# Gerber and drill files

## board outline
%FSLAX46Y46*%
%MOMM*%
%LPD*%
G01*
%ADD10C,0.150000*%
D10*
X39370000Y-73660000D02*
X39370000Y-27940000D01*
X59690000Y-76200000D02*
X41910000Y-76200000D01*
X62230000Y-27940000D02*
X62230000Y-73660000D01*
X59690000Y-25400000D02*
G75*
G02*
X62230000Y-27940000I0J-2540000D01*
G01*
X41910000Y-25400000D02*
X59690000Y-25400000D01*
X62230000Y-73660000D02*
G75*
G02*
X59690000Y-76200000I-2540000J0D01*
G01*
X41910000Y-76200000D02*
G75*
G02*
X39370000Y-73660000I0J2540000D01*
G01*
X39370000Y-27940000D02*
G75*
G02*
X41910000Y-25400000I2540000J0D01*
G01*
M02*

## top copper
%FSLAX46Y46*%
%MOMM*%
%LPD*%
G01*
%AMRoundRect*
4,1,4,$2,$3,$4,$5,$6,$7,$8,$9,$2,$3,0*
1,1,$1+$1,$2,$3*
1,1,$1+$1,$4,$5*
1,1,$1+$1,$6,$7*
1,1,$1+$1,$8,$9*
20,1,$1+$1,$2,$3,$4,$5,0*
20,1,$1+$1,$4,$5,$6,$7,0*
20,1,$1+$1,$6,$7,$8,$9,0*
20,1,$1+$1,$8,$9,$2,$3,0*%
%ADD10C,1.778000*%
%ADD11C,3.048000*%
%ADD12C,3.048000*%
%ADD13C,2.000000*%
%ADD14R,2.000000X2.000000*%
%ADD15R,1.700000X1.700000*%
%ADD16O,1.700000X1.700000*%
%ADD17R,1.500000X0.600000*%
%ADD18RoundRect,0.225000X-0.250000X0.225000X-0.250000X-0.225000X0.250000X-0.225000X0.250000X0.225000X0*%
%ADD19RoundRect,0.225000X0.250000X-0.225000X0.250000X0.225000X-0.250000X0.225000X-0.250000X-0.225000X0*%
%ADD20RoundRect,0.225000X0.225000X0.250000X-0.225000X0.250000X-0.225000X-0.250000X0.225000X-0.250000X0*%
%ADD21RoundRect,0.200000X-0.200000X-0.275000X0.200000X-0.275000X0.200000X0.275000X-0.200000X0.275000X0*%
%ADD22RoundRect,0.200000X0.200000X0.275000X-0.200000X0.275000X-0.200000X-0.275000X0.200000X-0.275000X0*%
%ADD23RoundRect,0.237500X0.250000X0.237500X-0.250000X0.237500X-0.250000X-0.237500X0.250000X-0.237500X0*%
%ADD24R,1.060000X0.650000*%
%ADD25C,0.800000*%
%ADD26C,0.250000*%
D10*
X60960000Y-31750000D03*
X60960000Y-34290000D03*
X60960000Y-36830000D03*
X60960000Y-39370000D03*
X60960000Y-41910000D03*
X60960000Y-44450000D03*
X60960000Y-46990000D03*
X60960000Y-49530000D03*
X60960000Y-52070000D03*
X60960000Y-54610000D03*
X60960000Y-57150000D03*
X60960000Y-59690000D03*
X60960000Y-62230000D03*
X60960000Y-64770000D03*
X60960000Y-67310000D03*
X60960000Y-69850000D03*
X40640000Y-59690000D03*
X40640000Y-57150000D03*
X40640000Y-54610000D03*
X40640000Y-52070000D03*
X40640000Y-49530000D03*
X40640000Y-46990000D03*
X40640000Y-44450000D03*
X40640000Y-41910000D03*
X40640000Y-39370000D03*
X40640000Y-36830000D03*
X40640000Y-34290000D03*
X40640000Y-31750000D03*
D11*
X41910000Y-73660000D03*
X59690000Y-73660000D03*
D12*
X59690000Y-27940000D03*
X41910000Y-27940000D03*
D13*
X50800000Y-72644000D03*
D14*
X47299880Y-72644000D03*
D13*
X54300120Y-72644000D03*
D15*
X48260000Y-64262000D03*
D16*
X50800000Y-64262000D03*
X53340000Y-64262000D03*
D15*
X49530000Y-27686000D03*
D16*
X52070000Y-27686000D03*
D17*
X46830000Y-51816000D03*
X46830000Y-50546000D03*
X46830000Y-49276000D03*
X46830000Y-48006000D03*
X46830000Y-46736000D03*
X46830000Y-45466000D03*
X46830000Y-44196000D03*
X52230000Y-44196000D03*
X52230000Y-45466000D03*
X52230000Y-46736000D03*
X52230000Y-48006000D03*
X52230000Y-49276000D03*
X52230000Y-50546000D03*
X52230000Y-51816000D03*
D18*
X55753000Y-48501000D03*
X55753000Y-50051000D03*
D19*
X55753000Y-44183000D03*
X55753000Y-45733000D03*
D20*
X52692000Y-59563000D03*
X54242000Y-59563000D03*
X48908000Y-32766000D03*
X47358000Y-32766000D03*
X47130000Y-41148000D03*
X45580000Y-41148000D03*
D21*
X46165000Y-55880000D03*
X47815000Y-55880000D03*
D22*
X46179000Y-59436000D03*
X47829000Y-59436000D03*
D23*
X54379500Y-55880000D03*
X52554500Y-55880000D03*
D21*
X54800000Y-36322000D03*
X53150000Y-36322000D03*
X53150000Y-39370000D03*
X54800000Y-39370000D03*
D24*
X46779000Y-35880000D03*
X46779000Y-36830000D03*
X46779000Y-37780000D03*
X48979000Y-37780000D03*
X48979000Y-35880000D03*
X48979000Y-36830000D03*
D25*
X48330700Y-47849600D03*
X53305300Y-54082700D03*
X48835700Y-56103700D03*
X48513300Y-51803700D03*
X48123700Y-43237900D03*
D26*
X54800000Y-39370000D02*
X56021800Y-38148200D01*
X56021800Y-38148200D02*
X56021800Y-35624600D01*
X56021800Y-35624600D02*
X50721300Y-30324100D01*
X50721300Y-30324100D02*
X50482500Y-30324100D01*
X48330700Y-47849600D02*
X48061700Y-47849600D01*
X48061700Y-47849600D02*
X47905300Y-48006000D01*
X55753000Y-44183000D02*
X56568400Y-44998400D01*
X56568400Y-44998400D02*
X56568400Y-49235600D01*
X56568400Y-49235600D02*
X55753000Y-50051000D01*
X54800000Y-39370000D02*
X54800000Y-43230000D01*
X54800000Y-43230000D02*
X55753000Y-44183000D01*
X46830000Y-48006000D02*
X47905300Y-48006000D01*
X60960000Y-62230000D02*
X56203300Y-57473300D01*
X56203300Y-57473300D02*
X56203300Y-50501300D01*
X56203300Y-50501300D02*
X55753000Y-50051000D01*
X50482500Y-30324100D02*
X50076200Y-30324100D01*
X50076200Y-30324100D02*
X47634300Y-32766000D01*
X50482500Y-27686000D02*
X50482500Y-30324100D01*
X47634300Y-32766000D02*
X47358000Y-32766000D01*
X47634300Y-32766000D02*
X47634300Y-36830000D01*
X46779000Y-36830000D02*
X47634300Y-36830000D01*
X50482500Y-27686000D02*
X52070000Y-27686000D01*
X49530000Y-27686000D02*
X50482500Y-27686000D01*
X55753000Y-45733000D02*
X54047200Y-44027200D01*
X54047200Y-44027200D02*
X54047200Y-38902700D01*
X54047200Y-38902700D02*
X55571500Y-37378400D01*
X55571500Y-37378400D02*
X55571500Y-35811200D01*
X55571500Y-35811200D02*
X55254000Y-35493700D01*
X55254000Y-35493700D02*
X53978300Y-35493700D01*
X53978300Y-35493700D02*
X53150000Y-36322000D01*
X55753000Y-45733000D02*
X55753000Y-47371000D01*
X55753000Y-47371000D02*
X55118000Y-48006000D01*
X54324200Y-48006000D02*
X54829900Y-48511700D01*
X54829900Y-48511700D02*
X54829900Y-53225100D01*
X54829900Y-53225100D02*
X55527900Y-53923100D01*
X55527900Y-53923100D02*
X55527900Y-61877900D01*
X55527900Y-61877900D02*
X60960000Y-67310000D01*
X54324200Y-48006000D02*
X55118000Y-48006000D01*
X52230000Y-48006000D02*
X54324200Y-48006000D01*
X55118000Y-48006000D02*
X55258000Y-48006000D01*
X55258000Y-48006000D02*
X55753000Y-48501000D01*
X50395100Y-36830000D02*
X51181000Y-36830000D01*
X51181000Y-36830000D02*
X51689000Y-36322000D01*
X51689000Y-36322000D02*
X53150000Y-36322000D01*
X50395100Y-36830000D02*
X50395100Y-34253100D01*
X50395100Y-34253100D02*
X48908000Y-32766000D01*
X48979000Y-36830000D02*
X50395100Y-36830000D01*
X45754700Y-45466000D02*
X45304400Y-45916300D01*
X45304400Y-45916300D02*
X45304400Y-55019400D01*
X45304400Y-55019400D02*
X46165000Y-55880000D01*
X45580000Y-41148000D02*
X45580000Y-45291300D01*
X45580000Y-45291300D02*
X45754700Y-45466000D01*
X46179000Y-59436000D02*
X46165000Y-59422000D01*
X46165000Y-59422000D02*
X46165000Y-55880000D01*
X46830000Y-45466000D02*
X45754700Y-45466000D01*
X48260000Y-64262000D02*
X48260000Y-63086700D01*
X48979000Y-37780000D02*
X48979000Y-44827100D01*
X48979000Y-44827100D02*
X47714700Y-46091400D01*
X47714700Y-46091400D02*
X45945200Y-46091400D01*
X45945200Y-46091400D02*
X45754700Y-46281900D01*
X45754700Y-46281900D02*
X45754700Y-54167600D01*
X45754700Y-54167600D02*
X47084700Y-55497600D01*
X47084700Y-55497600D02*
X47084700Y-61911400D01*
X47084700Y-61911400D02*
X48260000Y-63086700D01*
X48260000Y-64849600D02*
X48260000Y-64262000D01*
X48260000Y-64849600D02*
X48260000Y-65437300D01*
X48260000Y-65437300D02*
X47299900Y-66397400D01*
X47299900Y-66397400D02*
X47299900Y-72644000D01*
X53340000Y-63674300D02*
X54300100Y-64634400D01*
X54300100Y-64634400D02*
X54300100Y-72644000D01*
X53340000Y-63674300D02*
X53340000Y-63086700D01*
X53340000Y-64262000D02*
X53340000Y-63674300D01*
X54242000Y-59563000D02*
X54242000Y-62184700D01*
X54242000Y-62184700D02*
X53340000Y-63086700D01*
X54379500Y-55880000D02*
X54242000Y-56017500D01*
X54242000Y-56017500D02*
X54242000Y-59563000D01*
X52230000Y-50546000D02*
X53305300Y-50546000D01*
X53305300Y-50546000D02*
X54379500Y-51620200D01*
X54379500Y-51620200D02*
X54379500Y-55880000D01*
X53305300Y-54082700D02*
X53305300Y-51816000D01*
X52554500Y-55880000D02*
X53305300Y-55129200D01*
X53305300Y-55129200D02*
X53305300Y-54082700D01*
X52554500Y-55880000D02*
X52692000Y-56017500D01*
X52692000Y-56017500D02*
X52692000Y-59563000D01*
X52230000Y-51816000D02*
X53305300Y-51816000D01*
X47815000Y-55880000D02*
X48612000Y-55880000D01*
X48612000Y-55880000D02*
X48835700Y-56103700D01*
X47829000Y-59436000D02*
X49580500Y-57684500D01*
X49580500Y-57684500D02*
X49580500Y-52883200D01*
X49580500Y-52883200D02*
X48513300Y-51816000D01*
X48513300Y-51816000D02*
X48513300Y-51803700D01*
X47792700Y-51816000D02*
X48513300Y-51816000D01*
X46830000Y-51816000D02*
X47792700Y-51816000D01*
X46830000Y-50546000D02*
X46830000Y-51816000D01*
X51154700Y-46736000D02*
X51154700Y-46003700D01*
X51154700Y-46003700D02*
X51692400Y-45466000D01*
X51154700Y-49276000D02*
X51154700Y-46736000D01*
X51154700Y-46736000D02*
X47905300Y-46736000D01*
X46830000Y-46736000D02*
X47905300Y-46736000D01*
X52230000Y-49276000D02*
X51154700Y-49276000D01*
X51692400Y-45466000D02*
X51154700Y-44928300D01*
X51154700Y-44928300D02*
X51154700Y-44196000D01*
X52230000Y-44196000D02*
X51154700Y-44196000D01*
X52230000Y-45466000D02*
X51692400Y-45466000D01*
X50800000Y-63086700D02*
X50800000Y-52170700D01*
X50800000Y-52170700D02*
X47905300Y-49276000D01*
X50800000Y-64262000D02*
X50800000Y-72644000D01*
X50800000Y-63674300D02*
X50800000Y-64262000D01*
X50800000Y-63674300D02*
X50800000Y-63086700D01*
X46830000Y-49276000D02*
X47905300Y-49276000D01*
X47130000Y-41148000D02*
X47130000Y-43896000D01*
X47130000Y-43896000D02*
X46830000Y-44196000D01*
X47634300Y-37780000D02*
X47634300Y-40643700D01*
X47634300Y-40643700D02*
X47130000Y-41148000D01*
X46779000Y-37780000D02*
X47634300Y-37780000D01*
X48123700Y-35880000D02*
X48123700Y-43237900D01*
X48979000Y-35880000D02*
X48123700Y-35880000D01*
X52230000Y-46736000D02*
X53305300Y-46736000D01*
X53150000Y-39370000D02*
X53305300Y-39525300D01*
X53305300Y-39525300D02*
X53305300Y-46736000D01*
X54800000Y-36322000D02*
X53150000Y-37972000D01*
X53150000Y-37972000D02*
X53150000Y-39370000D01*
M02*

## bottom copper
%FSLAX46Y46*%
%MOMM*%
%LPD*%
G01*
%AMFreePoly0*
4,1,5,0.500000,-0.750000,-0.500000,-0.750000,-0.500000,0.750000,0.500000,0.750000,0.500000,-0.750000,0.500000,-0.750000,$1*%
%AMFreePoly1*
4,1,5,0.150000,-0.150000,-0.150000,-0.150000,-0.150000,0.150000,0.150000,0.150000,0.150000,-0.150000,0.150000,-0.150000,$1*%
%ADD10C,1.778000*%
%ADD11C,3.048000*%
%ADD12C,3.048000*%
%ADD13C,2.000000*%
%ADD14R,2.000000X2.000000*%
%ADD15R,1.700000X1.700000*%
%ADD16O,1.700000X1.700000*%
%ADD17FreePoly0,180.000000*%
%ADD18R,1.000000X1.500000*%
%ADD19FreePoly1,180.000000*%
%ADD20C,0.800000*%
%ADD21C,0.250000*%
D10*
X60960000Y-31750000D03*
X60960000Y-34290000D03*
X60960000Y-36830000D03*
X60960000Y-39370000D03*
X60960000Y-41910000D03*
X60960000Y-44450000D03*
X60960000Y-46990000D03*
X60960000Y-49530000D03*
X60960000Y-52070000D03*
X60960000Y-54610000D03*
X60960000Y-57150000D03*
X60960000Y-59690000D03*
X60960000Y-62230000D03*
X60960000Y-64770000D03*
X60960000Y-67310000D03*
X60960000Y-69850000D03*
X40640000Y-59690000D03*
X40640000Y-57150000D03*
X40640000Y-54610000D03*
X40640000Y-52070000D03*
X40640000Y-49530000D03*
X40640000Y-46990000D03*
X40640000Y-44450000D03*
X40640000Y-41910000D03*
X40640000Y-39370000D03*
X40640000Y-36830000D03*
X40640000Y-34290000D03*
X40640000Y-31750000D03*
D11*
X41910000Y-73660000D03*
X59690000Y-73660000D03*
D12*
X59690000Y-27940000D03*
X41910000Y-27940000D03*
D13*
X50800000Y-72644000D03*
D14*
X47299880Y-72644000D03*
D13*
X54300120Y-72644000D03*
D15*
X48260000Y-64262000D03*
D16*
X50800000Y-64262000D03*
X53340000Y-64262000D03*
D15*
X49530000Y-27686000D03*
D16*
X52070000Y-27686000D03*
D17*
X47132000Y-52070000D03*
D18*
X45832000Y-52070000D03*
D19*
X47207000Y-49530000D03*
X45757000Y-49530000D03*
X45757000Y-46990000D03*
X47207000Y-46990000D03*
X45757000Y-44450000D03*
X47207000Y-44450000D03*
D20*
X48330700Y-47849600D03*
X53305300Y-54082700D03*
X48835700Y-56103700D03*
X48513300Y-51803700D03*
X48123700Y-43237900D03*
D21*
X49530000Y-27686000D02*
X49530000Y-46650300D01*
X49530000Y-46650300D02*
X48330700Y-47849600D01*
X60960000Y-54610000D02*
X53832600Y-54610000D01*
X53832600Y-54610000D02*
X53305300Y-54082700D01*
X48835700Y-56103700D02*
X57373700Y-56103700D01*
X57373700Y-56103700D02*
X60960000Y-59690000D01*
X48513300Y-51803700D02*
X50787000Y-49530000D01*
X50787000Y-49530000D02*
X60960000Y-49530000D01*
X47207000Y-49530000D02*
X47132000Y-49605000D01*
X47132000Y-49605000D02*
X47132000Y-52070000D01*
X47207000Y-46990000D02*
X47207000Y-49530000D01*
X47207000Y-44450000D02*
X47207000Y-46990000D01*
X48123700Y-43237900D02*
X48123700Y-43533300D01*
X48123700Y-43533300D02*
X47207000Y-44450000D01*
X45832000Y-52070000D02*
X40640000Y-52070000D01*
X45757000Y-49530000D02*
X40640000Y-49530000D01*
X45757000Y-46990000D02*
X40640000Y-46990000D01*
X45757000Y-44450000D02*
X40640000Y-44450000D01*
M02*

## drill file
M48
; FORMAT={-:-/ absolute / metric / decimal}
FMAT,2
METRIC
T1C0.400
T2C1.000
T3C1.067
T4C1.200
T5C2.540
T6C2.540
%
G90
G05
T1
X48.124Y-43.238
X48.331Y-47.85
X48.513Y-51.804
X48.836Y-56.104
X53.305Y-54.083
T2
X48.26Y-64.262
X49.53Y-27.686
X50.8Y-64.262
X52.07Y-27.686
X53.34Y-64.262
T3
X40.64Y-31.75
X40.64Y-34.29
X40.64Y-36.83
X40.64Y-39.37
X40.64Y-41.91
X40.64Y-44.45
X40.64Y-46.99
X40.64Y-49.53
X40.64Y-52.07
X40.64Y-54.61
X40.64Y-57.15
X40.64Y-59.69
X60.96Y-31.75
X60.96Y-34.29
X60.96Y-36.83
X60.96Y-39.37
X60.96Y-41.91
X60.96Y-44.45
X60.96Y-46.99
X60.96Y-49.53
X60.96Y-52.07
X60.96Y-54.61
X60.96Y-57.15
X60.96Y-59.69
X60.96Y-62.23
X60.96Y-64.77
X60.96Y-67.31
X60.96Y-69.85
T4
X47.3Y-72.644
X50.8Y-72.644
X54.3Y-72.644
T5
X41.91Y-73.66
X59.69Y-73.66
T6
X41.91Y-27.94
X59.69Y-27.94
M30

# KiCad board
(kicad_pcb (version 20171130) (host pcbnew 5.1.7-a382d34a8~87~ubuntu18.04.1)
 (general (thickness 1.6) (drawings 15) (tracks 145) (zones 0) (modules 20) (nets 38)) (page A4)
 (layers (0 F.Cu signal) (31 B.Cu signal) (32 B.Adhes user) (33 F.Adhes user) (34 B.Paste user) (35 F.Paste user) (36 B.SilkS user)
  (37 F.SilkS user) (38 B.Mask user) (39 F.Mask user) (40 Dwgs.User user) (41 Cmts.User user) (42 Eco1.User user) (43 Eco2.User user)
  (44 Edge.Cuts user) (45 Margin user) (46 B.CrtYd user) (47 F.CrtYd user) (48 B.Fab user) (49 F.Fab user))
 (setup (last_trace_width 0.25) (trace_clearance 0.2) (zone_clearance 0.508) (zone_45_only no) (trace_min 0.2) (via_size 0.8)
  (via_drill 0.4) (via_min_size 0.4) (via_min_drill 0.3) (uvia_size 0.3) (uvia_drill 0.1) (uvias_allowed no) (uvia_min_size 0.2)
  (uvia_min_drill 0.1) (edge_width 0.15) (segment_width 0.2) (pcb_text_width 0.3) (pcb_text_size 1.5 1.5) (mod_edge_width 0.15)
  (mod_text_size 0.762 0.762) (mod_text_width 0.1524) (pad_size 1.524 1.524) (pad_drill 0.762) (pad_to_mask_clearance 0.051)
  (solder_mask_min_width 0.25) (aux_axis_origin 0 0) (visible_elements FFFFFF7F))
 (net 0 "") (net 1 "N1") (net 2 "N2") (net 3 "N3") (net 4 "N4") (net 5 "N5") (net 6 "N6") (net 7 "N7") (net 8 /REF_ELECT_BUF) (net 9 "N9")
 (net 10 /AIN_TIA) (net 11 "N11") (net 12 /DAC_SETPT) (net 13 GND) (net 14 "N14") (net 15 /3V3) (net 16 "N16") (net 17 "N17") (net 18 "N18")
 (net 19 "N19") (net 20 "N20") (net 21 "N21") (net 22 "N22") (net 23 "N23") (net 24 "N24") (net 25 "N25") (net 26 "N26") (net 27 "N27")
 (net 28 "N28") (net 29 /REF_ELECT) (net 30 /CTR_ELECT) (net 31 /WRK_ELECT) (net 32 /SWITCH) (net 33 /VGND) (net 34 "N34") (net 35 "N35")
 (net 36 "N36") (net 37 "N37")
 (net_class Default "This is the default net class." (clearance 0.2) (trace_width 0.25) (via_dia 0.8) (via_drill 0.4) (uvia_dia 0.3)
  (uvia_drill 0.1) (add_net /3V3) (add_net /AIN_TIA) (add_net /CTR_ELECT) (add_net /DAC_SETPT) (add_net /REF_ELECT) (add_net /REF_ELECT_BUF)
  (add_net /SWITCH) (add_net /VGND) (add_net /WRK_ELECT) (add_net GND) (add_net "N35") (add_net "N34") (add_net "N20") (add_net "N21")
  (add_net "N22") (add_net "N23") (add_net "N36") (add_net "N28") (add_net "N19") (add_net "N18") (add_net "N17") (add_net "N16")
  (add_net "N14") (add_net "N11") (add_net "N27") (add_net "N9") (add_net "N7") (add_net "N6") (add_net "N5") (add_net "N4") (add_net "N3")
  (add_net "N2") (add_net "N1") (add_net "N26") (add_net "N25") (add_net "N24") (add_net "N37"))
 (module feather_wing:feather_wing (layer F.Cu) (at 50.8 50.8)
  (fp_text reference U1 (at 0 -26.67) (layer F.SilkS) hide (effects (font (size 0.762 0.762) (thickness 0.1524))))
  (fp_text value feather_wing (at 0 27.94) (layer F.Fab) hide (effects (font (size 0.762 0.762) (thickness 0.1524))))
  (pad 28 thru_hole circle (at 10.16 -19.05) (size 1.778 1.778) (drill 1.0668) (layers *.Cu *.Mask) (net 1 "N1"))
  (pad 27 thru_hole circle (at 10.16 -16.51) (size 1.778 1.778) (drill 1.0668) (layers *.Cu *.Mask) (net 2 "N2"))
  (pad 26 thru_hole circle (at 10.16 -13.97) (size 1.778 1.778) (drill 1.0668) (layers *.Cu *.Mask) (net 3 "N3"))
  (pad 25 thru_hole circle (at 10.16 -11.43) (size 1.778 1.778) (drill 1.0668) (layers *.Cu *.Mask) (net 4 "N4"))
  (pad 24 thru_hole circle (at 10.16 -8.89) (size 1.778 1.778) (drill 1.0668) (layers *.Cu *.Mask) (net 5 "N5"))
  (pad 23 thru_hole circle (at 10.16 -6.35) (size 1.778 1.778) (drill 1.0668) (layers *.Cu *.Mask) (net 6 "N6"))
  (pad 22 thru_hole circle (at 10.16 -3.81) (size 1.778 1.778) (drill 1.0668) (layers *.Cu *.Mask) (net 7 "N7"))
  (pad 21 thru_hole circle (at 10.16 -1.27) (size 1.778 1.778) (drill 1.0668) (layers *.Cu *.Mask) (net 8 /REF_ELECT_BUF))
  (pad 20 thru_hole circle (at 10.16 1.27) (size 1.778 1.778) (drill 1.0668) (layers *.Cu *.Mask) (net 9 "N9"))
  (pad 19 thru_hole circle (at 10.16 3.81) (size 1.778 1.778) (drill 1.0668) (layers *.Cu *.Mask) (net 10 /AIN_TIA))
  (pad 18 thru_hole circle (at 10.16 6.35) (size 1.778 1.778) (drill 1.0668) (layers *.Cu *.Mask) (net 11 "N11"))
  (pad 17 thru_hole circle (at 10.16 8.89) (size 1.778 1.778) (drill 1.0668) (layers *.Cu *.Mask) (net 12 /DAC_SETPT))
  (pad 16 thru_hole circle (at 10.16 11.43) (size 1.778 1.778) (drill 1.0668) (layers *.Cu *.Mask) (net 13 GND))
  (pad 15 thru_hole circle (at 10.16 13.97) (size 1.778 1.778) (drill 1.0668) (layers *.Cu *.Mask) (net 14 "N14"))
  (pad 14 thru_hole circle (at 10.16 16.51) (size 1.778 1.778) (drill 1.0668) (layers *.Cu *.Mask) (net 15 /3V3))
  (pad 13 thru_hole circle (at 10.16 19.05) (size 1.778 1.778) (drill 1.0668) (layers *.Cu *.Mask) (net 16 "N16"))
  (pad 12 thru_hole circle (at -10.16 8.89) (size 1.778 1.778) (drill 1.0668) (layers *.Cu *.Mask) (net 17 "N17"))
  (pad 11 thru_hole circle (at -10.16 6.35) (size 1.778 1.778) (drill 1.0668) (layers *.Cu *.Mask) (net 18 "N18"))
  (pad 10 thru_hole circle (at -10.16 3.81) (size 1.778 1.778) (drill 1.0668) (layers *.Cu *.Mask) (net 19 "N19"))
  (pad 9 thru_hole circle (at -10.16 1.27) (size 1.778 1.778) (drill 1.0668) (layers *.Cu *.Mask) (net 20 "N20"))
  (pad 8 thru_hole circle (at -10.16 -1.27) (size 1.778 1.778) (drill 1.0668) (layers *.Cu *.Mask) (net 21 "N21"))
  (pad 7 thru_hole circle (at -10.16 -3.81) (size 1.778 1.778) (drill 1.0668) (layers *.Cu *.Mask) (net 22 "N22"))
  (pad 6 thru_hole circle (at -10.16 -6.35) (size 1.778 1.778) (drill 1.0668) (layers *.Cu *.Mask) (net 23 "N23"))
  (pad 5 thru_hole circle (at -10.16 -8.89) (size 1.778 1.778) (drill 1.0668) (layers *.Cu *.Mask) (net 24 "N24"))
  (pad 4 thru_hole circle (at -10.16 -11.43) (size 1.778 1.778) (drill 1.0668) (layers *.Cu *.Mask) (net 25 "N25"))
  (pad 3 thru_hole circle (at -10.16 -13.97) (size 1.778 1.778) (drill 1.0668) (layers *.Cu *.Mask) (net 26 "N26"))
  (pad 2 thru_hole circle (at -10.16 -16.51) (size 1.778 1.778) (drill 1.0668) (layers *.Cu *.Mask) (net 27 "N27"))
  (pad 1 thru_hole circle (at -10.16 -19.05) (size 1.778 1.778) (drill 1.0668) (layers *.Cu *.Mask) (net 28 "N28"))
  (pad "" thru_hole circle (at -8.89 22.86) (size 3.048 3.048) (drill 2.54) (layers *.Cu *.Mask))
  (pad "" thru_hole circle (at 8.89 22.86) (size 3.048 3.048) (drill 2.54) (layers *.Cu *.Mask))
  (pad "" np_thru_hole circle (at 8.89 -22.86) (size 3.048 3.048) (drill 2.54) (layers *.Cu *.Mask))
  (pad "" np_thru_hole circle (at -8.89 -22.86) (size 3.048 3.048) (drill 2.54) (layers *.Cu *.Mask)))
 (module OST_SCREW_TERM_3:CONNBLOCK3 (layer F.Cu) (at 50.8 72.644)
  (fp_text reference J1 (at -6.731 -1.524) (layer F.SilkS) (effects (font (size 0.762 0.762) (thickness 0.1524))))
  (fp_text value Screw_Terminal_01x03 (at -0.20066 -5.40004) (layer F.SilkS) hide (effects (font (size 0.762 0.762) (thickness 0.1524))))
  (pad 2 thru_hole circle (at 0 0) (size 2 2) (drill 1.2) (layers *.Cu *.Mask) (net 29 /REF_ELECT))
  (pad 1 thru_hole rect (at -3.50012 0) (size 2 2) (drill 1.2) (layers *.Cu *.Mask) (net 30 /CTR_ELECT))
  (pad 3 thru_hole circle (at 3.50012 0) (size 2 2) (drill 1.2) (layers *.Cu *.Mask) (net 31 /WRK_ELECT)))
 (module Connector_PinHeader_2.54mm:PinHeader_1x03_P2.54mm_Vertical (layer F.Cu) (at 48.26 64.262 90)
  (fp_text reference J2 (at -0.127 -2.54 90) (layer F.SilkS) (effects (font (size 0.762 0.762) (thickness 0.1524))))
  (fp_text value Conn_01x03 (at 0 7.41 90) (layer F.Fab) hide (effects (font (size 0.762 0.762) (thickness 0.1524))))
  (pad 1 thru_hole rect (at 0 0 90) (size 1.7 1.7) (drill 1) (layers *.Cu *.Mask) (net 30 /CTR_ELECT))
  (pad 2 thru_hole oval (at 0 2.54 90) (size 1.7 1.7) (drill 1) (layers *.Cu *.Mask) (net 29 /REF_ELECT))
  (pad 3 thru_hole oval (at 0 5.08 90) (size 1.7 1.7) (drill 1) (layers *.Cu *.Mask) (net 31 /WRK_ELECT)))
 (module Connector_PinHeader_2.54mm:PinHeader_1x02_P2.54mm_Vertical (layer F.Cu) (at 49.53 27.686 90)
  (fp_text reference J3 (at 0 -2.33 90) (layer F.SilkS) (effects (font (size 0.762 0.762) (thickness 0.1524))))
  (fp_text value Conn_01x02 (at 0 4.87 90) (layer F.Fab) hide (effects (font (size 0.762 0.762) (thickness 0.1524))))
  (pad 1 thru_hole rect (at 0 0 90) (size 1.7 1.7) (drill 1) (layers *.Cu *.Mask) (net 13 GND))
  (pad 2 thru_hole oval (at 0 2.54 90) (size 1.7 1.7) (drill 1) (layers *.Cu *.Mask) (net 13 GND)))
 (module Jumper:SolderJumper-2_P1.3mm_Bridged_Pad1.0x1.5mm (layer B.Cu) (at 46.482 52.07 180)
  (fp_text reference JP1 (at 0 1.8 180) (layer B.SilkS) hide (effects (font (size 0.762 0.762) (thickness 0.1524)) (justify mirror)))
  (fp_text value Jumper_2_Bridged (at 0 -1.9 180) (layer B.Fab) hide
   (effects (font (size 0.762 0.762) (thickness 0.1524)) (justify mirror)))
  (pad 1 smd custom (at -0.65 0 180) (size 1 1.5) (layers B.Cu B.Mask) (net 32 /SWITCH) (options (clearance outline) (anchor rect))
   (primitives))
  (pad 2 smd rect (at 0.65 0 180) (size 1 1.5) (layers B.Cu B.Mask) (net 20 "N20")))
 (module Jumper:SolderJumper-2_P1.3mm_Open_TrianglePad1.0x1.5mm (layer B.Cu) (at 46.482 49.53 180)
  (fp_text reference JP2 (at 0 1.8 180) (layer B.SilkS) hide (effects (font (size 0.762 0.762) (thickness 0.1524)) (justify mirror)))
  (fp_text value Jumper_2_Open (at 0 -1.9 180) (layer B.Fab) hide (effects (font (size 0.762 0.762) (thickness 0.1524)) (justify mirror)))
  (pad 1 smd custom (at -0.725 0 180) (size 0.3 0.3) (layers B.Cu B.Mask) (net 32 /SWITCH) (zone_connect 0)
   (options (clearance outline) (anchor rect)) (primitives))
  (pad 2 smd custom (at 0.725 0 180) (size 0.3 0.3) (layers B.Cu B.Mask) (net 21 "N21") (zone_connect 0)
   (options (clearance outline) (anchor rect)) (primitives)))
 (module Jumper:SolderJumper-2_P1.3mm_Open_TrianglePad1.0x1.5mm (layer B.Cu) (at 46.482 46.99 180)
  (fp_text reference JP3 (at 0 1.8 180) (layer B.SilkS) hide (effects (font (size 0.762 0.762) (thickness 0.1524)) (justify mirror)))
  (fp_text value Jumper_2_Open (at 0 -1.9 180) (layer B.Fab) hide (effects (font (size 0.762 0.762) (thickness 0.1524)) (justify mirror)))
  (pad 2 smd custom (at 0.725 0 180) (size 0.3 0.3) (layers B.Cu B.Mask) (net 22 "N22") (zone_connect 0)
   (options (clearance outline) (anchor rect)) (primitives))
  (pad 1 smd custom (at -0.725 0 180) (size 0.3 0.3) (layers B.Cu B.Mask) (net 32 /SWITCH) (zone_connect 0)
   (options (clearance outline) (anchor rect)) (primitives)))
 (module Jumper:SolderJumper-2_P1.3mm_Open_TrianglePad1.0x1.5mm (layer B.Cu) (at 46.482 44.45 180)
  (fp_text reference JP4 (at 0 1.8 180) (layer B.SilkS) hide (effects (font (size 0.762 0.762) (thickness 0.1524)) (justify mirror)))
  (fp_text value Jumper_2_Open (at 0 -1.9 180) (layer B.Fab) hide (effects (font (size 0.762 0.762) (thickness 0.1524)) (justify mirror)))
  (pad 2 smd custom (at 0.725 0 180) (size 0.3 0.3) (layers B.Cu B.Mask) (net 23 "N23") (zone_connect 0)
   (options (clearance outline) (anchor rect)) (primitives))
  (pad 1 smd custom (at -0.725 0 180) (size 0.3 0.3) (layers B.Cu B.Mask) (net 32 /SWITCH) (zone_connect 0)
   (options (clearance outline) (anchor rect)) (primitives)))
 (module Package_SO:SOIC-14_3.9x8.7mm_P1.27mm (layer F.Cu) (at 49.53 48.006 180)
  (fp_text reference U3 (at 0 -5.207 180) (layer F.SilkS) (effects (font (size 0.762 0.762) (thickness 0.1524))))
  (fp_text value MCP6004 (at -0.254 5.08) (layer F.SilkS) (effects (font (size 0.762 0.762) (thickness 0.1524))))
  (pad 14 smd rect (at 2.7 -3.81 180) (size 1.5 0.6) (layers F.Cu F.Paste F.Mask) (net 8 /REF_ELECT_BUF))
  (pad 13 smd rect (at 2.7 -2.54 180) (size 1.5 0.6) (layers F.Cu F.Paste F.Mask) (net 8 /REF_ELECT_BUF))
  (pad 12 smd rect (at 2.7 -1.27 180) (size 1.5 0.6) (layers F.Cu F.Paste F.Mask) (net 29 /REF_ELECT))
  (pad 11 smd rect (at 2.7 0 180) (size 1.5 0.6) (layers F.Cu F.Paste F.Mask) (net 13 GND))
  (pad 10 smd rect (at 2.7 1.27 180) (size 1.5 0.6) (layers F.Cu F.Paste F.Mask) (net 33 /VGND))
  (pad 9 smd rect (at 2.7 2.54 180) (size 1.5 0.6) (layers F.Cu F.Paste F.Mask) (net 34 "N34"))
  (pad 8 smd rect (at 2.7 3.81 180) (size 1.5 0.6) (layers F.Cu F.Paste F.Mask) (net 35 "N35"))
  (pad 7 smd rect (at -2.7 3.81 180) (size 1.5 0.6) (layers F.Cu F.Paste F.Mask) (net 33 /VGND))
  (pad 6 smd rect (at -2.7 2.54 180) (size 1.5 0.6) (layers F.Cu F.Paste F.Mask) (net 33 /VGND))
  (pad 5 smd rect (at -2.7 1.27 180) (size 1.5 0.6) (layers F.Cu F.Paste F.Mask) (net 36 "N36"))
  (pad 4 smd rect (at -2.7 0 180) (size 1.5 0.6) (layers F.Cu F.Paste F.Mask) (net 15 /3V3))
  (pad 3 smd rect (at -2.7 -1.27 180) (size 1.5 0.6) (layers F.Cu F.Paste F.Mask) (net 33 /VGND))
  (pad 2 smd rect (at -2.7 -2.54 180) (size 1.5 0.6) (layers F.Cu F.Paste F.Mask) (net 31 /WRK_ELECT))
  (pad 1 smd rect (at -2.7 -3.81 180) (size 1.5 0.6) (layers F.Cu F.Paste F.Mask) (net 10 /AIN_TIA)))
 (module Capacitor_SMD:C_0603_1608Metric (layer F.Cu) (at 55.753 49.276 270)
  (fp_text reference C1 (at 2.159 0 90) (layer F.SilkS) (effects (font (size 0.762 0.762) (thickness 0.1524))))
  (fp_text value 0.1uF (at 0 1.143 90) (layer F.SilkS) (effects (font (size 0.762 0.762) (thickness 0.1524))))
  (pad 1 smd roundrect (at -0.775 0 270) (size 0.9 0.95) (layers F.Cu F.Paste F.Mask) (roundrect_rratio 0.25) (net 15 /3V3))
  (pad 2 smd roundrect (at 0.775 0 270) (size 0.9 0.95) (layers F.Cu F.Paste F.Mask) (roundrect_rratio 0.25) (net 13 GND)))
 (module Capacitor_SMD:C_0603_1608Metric (layer F.Cu) (at 55.753 44.958 90)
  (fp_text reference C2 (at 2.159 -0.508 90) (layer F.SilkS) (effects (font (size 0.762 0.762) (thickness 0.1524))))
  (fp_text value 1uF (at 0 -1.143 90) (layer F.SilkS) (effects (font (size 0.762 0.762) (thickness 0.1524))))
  (pad 2 smd roundrect (at 0.775 0 90) (size 0.9 0.95) (layers F.Cu F.Paste F.Mask) (roundrect_rratio 0.25) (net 13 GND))
  (pad 1 smd roundrect (at -0.775 0 90) (size 0.9 0.95) (layers F.Cu F.Paste F.Mask) (roundrect_rratio 0.25) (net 15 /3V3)))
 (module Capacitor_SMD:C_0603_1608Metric (layer F.Cu) (at 53.467 59.563 180)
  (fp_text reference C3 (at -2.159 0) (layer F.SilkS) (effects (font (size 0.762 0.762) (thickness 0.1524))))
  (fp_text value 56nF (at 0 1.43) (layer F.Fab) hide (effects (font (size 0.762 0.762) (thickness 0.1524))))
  (pad 2 smd roundrect (at 0.775 0 180) (size 0.9 0.95) (layers F.Cu F.Paste F.Mask) (roundrect_rratio 0.25) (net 10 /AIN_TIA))
  (pad 1 smd roundrect (at -0.775 0 180) (size 0.9 0.95) (layers F.Cu F.Paste F.Mask) (roundrect_rratio 0.25) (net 31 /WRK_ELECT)))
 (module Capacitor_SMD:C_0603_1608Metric (layer F.Cu) (at 48.133 32.766 180)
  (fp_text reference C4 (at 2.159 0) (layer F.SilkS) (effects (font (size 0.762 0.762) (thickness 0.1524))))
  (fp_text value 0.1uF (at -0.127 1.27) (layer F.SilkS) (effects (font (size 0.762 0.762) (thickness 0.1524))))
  (pad 1 smd roundrect (at -0.775 0 180) (size 0.9 0.95) (layers F.Cu F.Paste F.Mask) (roundrect_rratio 0.25) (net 15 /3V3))
  (pad 2 smd roundrect (at 0.775 0 180) (size 0.9 0.95) (layers F.Cu F.Paste F.Mask) (roundrect_rratio 0.25) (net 13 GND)))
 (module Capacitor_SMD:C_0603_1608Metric (layer F.Cu) (at 46.355 41.148 180)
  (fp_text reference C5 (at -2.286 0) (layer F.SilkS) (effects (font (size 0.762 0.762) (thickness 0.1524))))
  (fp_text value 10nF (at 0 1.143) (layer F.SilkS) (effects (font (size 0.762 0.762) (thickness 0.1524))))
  (pad 1 smd roundrect (at -0.775 0 180) (size 0.9 0.95) (layers F.Cu F.Paste F.Mask) (roundrect_rratio 0.25) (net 35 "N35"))
  (pad 2 smd roundrect (at 0.775 0 180) (size 0.9 0.95) (layers F.Cu F.Paste F.Mask) (roundrect_rratio 0.25) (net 34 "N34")))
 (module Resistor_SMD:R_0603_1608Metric (layer F.Cu) (at 46.99 55.88)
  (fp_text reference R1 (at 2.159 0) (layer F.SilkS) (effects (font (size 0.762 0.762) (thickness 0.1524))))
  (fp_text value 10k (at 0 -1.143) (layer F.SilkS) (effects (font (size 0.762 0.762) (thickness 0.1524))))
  (pad 1 smd roundrect (at -0.825 0) (size 0.8 0.95) (layers F.Cu F.Paste F.Mask) (roundrect_rratio 0.25) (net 34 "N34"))
  (pad 2 smd roundrect (at 0.825 0) (size 0.8 0.95) (layers F.Cu F.Paste F.Mask) (roundrect_rratio 0.25) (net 12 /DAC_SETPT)))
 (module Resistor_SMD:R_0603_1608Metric (layer F.Cu) (at 47.004 59.436 180)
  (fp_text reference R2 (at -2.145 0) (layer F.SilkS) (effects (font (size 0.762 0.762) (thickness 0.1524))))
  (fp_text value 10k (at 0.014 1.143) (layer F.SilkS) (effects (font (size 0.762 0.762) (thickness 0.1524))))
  (pad 2 smd roundrect (at 0.825 0 180) (size 0.8 0.95) (layers F.Cu F.Paste F.Mask) (roundrect_rratio 0.25) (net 34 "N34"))
  (pad 1 smd roundrect (at -0.825 0 180) (size 0.8 0.95) (layers F.Cu F.Paste F.Mask) (roundrect_rratio 0.25) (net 8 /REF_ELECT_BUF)))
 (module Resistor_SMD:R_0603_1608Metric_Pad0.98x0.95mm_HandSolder (layer F.Cu) (at 53.467 55.88 180)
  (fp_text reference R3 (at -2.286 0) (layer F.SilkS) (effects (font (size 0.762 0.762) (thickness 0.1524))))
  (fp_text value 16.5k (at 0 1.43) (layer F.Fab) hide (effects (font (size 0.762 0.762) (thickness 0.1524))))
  (pad 1 smd roundrect (at -0.9125 0 180) (size 0.975 0.95) (layers F.Cu F.Paste F.Mask) (roundrect_rratio 0.25) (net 31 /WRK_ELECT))
  (pad 2 smd roundrect (at 0.9125 0 180) (size 0.975 0.95) (layers F.Cu F.Paste F.Mask) (roundrect_rratio 0.25) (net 10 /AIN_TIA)))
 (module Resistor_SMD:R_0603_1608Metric (layer F.Cu) (at 53.975 36.322)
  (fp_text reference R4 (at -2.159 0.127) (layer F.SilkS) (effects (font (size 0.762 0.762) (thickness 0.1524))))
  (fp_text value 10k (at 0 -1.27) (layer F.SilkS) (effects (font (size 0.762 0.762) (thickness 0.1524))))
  (pad 2 smd roundrect (at 0.825 0) (size 0.8 0.95) (layers F.Cu F.Paste F.Mask) (roundrect_rratio 0.25) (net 36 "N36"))
  (pad 1 smd roundrect (at -0.825 0) (size 0.8 0.95) (layers F.Cu F.Paste F.Mask) (roundrect_rratio 0.25) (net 15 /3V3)))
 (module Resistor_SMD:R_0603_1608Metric (layer F.Cu) (at 53.975 39.37)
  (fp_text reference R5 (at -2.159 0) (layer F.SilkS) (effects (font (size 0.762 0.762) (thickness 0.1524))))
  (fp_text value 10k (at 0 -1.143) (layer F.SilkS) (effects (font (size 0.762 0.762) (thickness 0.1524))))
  (pad 1 smd roundrect (at -0.825 0) (size 0.8 0.95) (layers F.Cu F.Paste F.Mask) (roundrect_rratio 0.25) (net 36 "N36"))
  (pad 2 smd roundrect (at 0.825 0) (size 0.8 0.95) (layers F.Cu F.Paste F.Mask) (roundrect_rratio 0.25) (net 13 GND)))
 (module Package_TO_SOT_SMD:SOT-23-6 (layer F.Cu) (at 47.879 36.83)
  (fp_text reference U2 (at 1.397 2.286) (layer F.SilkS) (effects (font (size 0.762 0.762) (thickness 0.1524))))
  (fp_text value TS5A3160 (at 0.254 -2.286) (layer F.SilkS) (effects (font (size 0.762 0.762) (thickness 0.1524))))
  (pad 1 smd rect (at -1.1 -0.95) (size 1.06 0.65) (layers F.Cu F.Paste F.Mask) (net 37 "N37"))
  (pad 2 smd rect (at -1.1 0) (size 1.06 0.65) (layers F.Cu F.Paste F.Mask) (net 13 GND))
  (pad 3 smd rect (at -1.1 0.95) (size 1.06 0.65) (layers F.Cu F.Paste F.Mask) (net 35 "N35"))
  (pad 4 smd rect (at 1.1 0.95) (size 1.06 0.65) (layers F.Cu F.Paste F.Mask) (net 30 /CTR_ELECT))
  (pad 6 smd rect (at 1.1 -0.95) (size 1.06 0.65) (layers F.Cu F.Paste F.Mask) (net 32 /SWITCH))
  (pad 5 smd rect (at 1.1 0) (size 1.06 0.65) (layers F.Cu F.Paste F.Mask) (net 15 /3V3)))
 (gr_line (start 39.37 73.66) (end 39.37 27.94) (layer Edge.Cuts) (width 0.15))
 (gr_line (start 59.69 76.2) (end 41.91 76.2) (layer Edge.Cuts) (width 0.15))
 (gr_line (start 62.23 27.94) (end 62.23 73.66) (layer Edge.Cuts) (width 0.15))
 (gr_arc (start 59.69 27.94) (end 62.23 27.94) (angle -90) (layer Edge.Cuts) (width 0.15))
 (gr_line (start 41.91 25.4) (end 59.69 25.4) (layer Edge.Cuts) (width 0.15))
 (gr_arc (start 59.69 73.66) (end 59.69 76.2) (angle -90) (layer Edge.Cuts) (width 0.15))
 (gr_arc (start 41.91 73.66) (end 39.37 73.66) (angle -90) (layer Edge.Cuts) (width 0.15))
 (gr_arc (start 41.91 27.94) (end 41.91 25.4) (angle -90) (layer Edge.Cuts) (width 0.15))
 (segment (start 54.8 39.37) (end 56.0218 38.1482) (width 0.25) (layer F.Cu) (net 13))
 (segment (start 56.0218 38.1482) (end 56.0218 35.6246) (width 0.25) (layer F.Cu) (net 13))
 (segment (start 56.0218 35.6246) (end 50.7213 30.3241) (width 0.25) (layer F.Cu) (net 13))
 (segment (start 50.7213 30.3241) (end 50.4825 30.3241) (width 0.25) (layer F.Cu) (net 13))
 (segment (start 48.3307 47.8496) (end 48.0617 47.8496) (width 0.25) (layer F.Cu) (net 13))
 (segment (start 48.0617 47.8496) (end 47.9053 48.006) (width 0.25) (layer F.Cu) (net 13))
 (segment (start 49.53 27.686) (end 49.53 46.6503) (width 0.25) (layer B.Cu) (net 13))
 (segment (start 49.53 46.6503) (end 48.3307 47.8496) (width 0.25) (layer B.Cu) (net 13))
 (segment (start 55.753 44.183) (end 56.5684 44.9984) (width 0.25) (layer F.Cu) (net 13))
 (segment (start 56.5684 44.9984) (end 56.5684 49.2356) (width 0.25) (layer F.Cu) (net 13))
 (segment (start 56.5684 49.2356) (end 55.753 50.051) (width 0.25) (layer F.Cu) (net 13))
 (segment (start 54.8 39.37) (end 54.8 43.23) (width 0.25) (layer F.Cu) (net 13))
 (segment (start 54.8 43.23) (end 55.753 44.183) (width 0.25) (layer F.Cu) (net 13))
 (segment (start 46.83 48.006) (end 47.9053 48.006) (width 0.25) (layer F.Cu) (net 13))
 (segment (start 60.96 62.23) (end 56.2033 57.4733) (width 0.25) (layer F.Cu) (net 13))
 (segment (start 56.2033 57.4733) (end 56.2033 50.5013) (width 0.25) (layer F.Cu) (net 13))
 (segment (start 56.2033 50.5013) (end 55.753 50.051) (width 0.25) (layer F.Cu) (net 13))
 (segment (start 50.4825 30.3241) (end 50.0762 30.3241) (width 0.25) (layer F.Cu) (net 13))
 (segment (start 50.0762 30.3241) (end 47.6343 32.766) (width 0.25) (layer F.Cu) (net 13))
 (segment (start 50.4825 27.686) (end 50.4825 30.3241) (width 0.25) (layer F.Cu) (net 13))
 (segment (start 47.6343 32.766) (end 47.358 32.766) (width 0.25) (layer F.Cu) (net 13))
 (segment (start 47.6343 32.766) (end 47.6343 36.83) (width 0.25) (layer F.Cu) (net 13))
 (segment (start 46.779 36.83) (end 47.6343 36.83) (width 0.25) (layer F.Cu) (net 13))
 (segment (start 50.4825 27.686) (end 52.07 27.686) (width 0.25) (layer F.Cu) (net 13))
 (segment (start 49.53 27.686) (end 50.4825 27.686) (width 0.25) (layer F.Cu) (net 13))
 (via (at 48.3307 47.8496) (size 0.8) (layers F.Cu B.Cu) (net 13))
 (segment (start 55.753 45.733) (end 54.0472 44.0272) (width 0.25) (layer F.Cu) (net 15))
 (segment (start 54.0472 44.0272) (end 54.0472 38.9027) (width 0.25) (layer F.Cu) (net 15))
 (segment (start 54.0472 38.9027) (end 55.5715 37.3784) (width 0.25) (layer F.Cu) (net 15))
 (segment (start 55.5715 37.3784) (end 55.5715 35.8112) (width 0.25) (layer F.Cu) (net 15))
 (segment (start 55.5715 35.8112) (end 55.254 35.4937) (width 0.25) (layer F.Cu) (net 15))
 (segment (start 55.254 35.4937) (end 53.9783 35.4937) (width 0.25) (layer F.Cu) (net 15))
 (segment (start 53.9783 35.4937) (end 53.15 36.322) (width 0.25) (layer F.Cu) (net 15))
 (segment (start 55.753 45.733) (end 55.753 47.371) (width 0.25) (layer F.Cu) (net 15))
 (segment (start 55.753 47.371) (end 55.118 48.006) (width 0.25) (layer F.Cu) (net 15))
 (segment (start 54.3242 48.006) (end 54.8299 48.5117) (width 0.25) (layer F.Cu) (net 15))
 (segment (start 54.8299 48.5117) (end 54.8299 53.2251) (width 0.25) (layer F.Cu) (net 15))
 (segment (start 54.8299 53.2251) (end 55.5279 53.9231) (width 0.25) (layer F.Cu) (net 15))
 (segment (start 55.5279 53.9231) (end 55.5279 61.8779) (width 0.25) (layer F.Cu) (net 15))
 (segment (start 55.5279 61.8779) (end 60.96 67.31) (width 0.25) (layer F.Cu) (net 15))
 (segment (start 54.3242 48.006) (end 55.118 48.006) (width 0.25) (layer F.Cu) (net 15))
 (segment (start 52.23 48.006) (end 54.3242 48.006) (width 0.25) (layer F.Cu) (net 15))
 (segment (start 55.118 48.006) (end 55.258 48.006) (width 0.25) (layer F.Cu) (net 15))
 (segment (start 55.258 48.006) (end 55.753 48.501) (width 0.25) (layer F.Cu) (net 15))
 (segment (start 50.3951 36.83) (end 51.181 36.83) (width 0.25) (layer F.Cu) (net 15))
 (segment (start 51.181 36.83) (end 51.689 36.322) (width 0.25) (layer F.Cu) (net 15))
 (segment (start 51.689 36.322) (end 53.15 36.322) (width 0.25) (layer F.Cu) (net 15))
 (segment (start 50.3951 36.83) (end 50.3951 34.2531) (width 0.25) (layer F.Cu) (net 15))
 (segment (start 50.3951 34.2531) (end 48.908 32.766) (width 0.25) (layer F.Cu) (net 15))
 (segment (start 48.979 36.83) (end 50.3951 36.83) (width 0.25) (layer F.Cu) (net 15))
 (segment (start 45.7547 45.466) (end 45.3044 45.9163) (width 0.25) (layer F.Cu) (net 34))
 (segment (start 45.3044 45.9163) (end 45.3044 55.0194) (width 0.25) (layer F.Cu) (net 34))
 (segment (start 45.3044 55.0194) (end 46.165 55.88) (width 0.25) (layer F.Cu) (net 34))
 (segment (start 45.58 41.148) (end 45.58 45.2913) (width 0.25) (layer F.Cu) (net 34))
 (segment (start 45.58 45.2913) (end 45.7547 45.466) (width 0.25) (layer F.Cu) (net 34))
 (segment (start 46.179 59.436) (end 46.165 59.422) (width 0.25) (layer F.Cu) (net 34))
 (segment (start 46.165 59.422) (end 46.165 55.88) (width 0.25) (layer F.Cu) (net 34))
 (segment (start 46.83 45.466) (end 45.7547 45.466) (width 0.25) (layer F.Cu) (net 34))
 (segment (start 48.26 64.262) (end 48.26 63.0867) (width 0.25) (layer F.Cu) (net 30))
 (segment (start 48.979 37.78) (end 48.979 44.8271) (width 0.25) (layer F.Cu) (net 30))
 (segment (start 48.979 44.8271) (end 47.7147 46.0914) (width 0.25) (layer F.Cu) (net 30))
 (segment (start 47.7147 46.0914) (end 45.9452 46.0914) (width 0.25) (layer F.Cu) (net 30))
 (segment (start 45.9452 46.0914) (end 45.7547 46.2819) (width 0.25) (layer F.Cu) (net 30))
 (segment (start 45.7547 46.2819) (end 45.7547 54.1676) (width 0.25) (layer F.Cu) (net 30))
 (segment (start 45.7547 54.1676) (end 47.0847 55.4976) (width 0.25) (layer F.Cu) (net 30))
 (segment (start 47.0847 55.4976) (end 47.0847 61.9114) (width 0.25) (layer F.Cu) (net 30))
 (segment (start 47.0847 61.9114) (end 48.26 63.0867) (width 0.25) (layer F.Cu) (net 30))
 (segment (start 48.26 64.8496) (end 48.26 64.262) (width 0.25) (layer F.Cu) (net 30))
 (segment (start 48.26 64.8496) (end 48.26 65.4373) (width 0.25) (layer F.Cu) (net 30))
 (segment (start 48.26 65.4373) (end 47.2999 66.3974) (width 0.25) (layer F.Cu) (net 30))
 (segment (start 47.2999 66.3974) (end 47.2999 72.644) (width 0.25) (layer F.Cu) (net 30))
 (segment (start 53.34 63.6743) (end 54.3001 64.6344) (width 0.25) (layer F.Cu) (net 31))
 (segment (start 54.3001 64.6344) (end 54.3001 72.644) (width 0.25) (layer F.Cu) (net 31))
 (segment (start 53.34 63.6743) (end 53.34 63.0867) (width 0.25) (layer F.Cu) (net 31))
 (segment (start 53.34 64.262) (end 53.34 63.6743) (width 0.25) (layer F.Cu) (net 31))
 (segment (start 54.242 59.563) (end 54.242 62.1847) (width 0.25) (layer F.Cu) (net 31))
 (segment (start 54.242 62.1847) (end 53.34 63.0867) (width 0.25) (layer F.Cu) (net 31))
 (segment (start 54.3795 55.88) (end 54.242 56.0175) (width 0.25) (layer F.Cu) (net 31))
 (segment (start 54.242 56.0175) (end 54.242 59.563) (width 0.25) (layer F.Cu) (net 31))
 (segment (start 52.23 50.546) (end 53.3053 50.546) (width 0.25) (layer F.Cu) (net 31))
 (segment (start 53.3053 50.546) (end 54.3795 51.6202) (width 0.25) (layer F.Cu) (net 31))
 (segment (start 54.3795 51.6202) (end 54.3795 55.88) (width 0.25) (layer F.Cu) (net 31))
 (segment (start 60.96 54.61) (end 53.8326 54.61) (width 0.25) (layer B.Cu) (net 10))
 (segment (start 53.8326 54.61) (end 53.3053 54.0827) (width 0.25) (layer B.Cu) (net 10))
 (segment (start 53.3053 54.0827) (end 53.3053 51.816) (width 0.25) (layer F.Cu) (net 10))
 (segment (start 52.5545 55.88) (end 53.3053 55.1292) (width 0.25) (layer F.Cu) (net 10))
 (segment (start 53.3053 55.1292) (end 53.3053 54.0827) (width 0.25) (layer F.Cu) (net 10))
 (segment (start 52.5545 55.88) (end 52.692 56.0175) (width 0.25) (layer F.Cu) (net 10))
 (segment (start 52.692 56.0175) (end 52.692 59.563) (width 0.25) (layer F.Cu) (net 10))
 (segment (start 52.23 51.816) (end 53.3053 51.816) (width 0.25) (layer F.Cu) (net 10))
 (via (at 53.3053 54.0827) (size 0.8) (layers F.Cu B.Cu) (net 10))
 (segment (start 48.8357 56.1037) (end 57.3737 56.1037) (width 0.25) (layer B.Cu) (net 12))
 (segment (start 57.3737 56.1037) (end 60.96 59.69) (width 0.25) (layer B.Cu) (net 12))
 (segment (start 47.815 55.88) (end 48.612 55.88) (width 0.25) (layer F.Cu) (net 12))
 (segment (start 48.612 55.88) (end 48.8357 56.1037) (width 0.25) (layer F.Cu) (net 12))
 (via (at 48.8357 56.1037) (size 0.8) (layers F.Cu B.Cu) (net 12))
 (segment (start 47.829 59.436) (end 49.5805 57.6845) (width 0.25) (layer F.Cu) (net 8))
 (segment (start 49.5805 57.6845) (end 49.5805 52.8832) (width 0.25) (layer F.Cu) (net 8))
 (segment (start 49.5805 52.8832) (end 48.5133 51.816) (width 0.25) (layer F.Cu) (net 8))
 (segment (start 48.5133 51.816) (end 48.5133 51.8037) (width 0.25) (layer F.Cu) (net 8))
 (segment (start 47.7927 51.816) (end 48.5133 51.816) (width 0.25) (layer F.Cu) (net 8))
 (segment (start 48.5133 51.8037) (end 50.787 49.53) (width 0.25) (layer B.Cu) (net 8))
 (segment (start 50.787 49.53) (end 60.96 49.53) (width 0.25) (layer B.Cu) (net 8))
 (segment (start 46.83 51.816) (end 47.7927 51.816) (width 0.25) (layer F.Cu) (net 8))
 (segment (start 46.83 50.546) (end 46.83 51.816) (width 0.25) (layer F.Cu) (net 8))
 (via (at 48.5133 51.8037) (size 0.8) (layers F.Cu B.Cu) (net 8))
 (segment (start 51.1547 46.736) (end 51.1547 46.0037) (width 0.25) (layer F.Cu) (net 33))
 (segment (start 51.1547 46.0037) (end 51.6924 45.466) (width 0.25) (layer F.Cu) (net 33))
 (segment (start 51.1547 49.276) (end 51.1547 46.736) (width 0.25) (layer F.Cu) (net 33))
 (segment (start 51.1547 46.736) (end 47.9053 46.736) (width 0.25) (layer F.Cu) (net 33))
 (segment (start 46.83 46.736) (end 47.9053 46.736) (width 0.25) (layer F.Cu) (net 33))
 (segment (start 52.23 49.276) (end 51.1547 49.276) (width 0.25) (layer F.Cu) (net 33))
 (segment (start 51.6924 45.466) (end 51.1547 44.9283) (width 0.25) (layer F.Cu) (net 33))
 (segment (start 51.1547 44.9283) (end 51.1547 44.196) (width 0.25) (layer F.Cu) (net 33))
 (segment (start 52.23 44.196) (end 51.1547 44.196) (width 0.25) (layer F.Cu) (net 33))
 (segment (start 52.23 45.466) (end 51.6924 45.466) (width 0.25) (layer F.Cu) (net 33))
 (segment (start 50.8 63.0867) (end 50.8 52.1707) (width 0.25) (layer F.Cu) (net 29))
 (segment (start 50.8 52.1707) (end 47.9053 49.276) (width 0.25) (layer F.Cu) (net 29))
 (segment (start 50.8 64.262) (end 50.8 72.644) (width 0.25) (layer F.Cu) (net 29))
 (segment (start 50.8 63.6743) (end 50.8 64.262) (width 0.25) (layer F.Cu) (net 29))
 (segment (start 50.8 63.6743) (end 50.8 63.0867) (width 0.25) (layer F.Cu) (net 29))
 (segment (start 46.83 49.276) (end 47.9053 49.276) (width 0.25) (layer F.Cu) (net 29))
 (segment (start 47.13 41.148) (end 47.13 43.896) (width 0.25) (layer F.Cu) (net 35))
 (segment (start 47.13 43.896) (end 46.83 44.196) (width 0.25) (layer F.Cu) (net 35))
 (segment (start 47.6343 37.78) (end 47.6343 40.6437) (width 0.25) (layer F.Cu) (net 35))
 (segment (start 47.6343 40.6437) (end 47.13 41.148) (width 0.25) (layer F.Cu) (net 35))
 (segment (start 46.779 37.78) (end 47.6343 37.78) (width 0.25) (layer F.Cu) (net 35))
 (segment (start 47.207 49.53) (end 47.132 49.605) (width 0.25) (layer B.Cu) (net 32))
 (segment (start 47.132 49.605) (end 47.132 52.07) (width 0.25) (layer B.Cu) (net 32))
 (segment (start 47.207 46.99) (end 47.207 49.53) (width 0.25) (layer B.Cu) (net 32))
 (segment (start 47.207 44.45) (end 47.207 46.99) (width 0.25) (layer B.Cu) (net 32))
 (segment (start 48.1237 43.2379) (end 48.1237 43.5333) (width 0.25) (layer B.Cu) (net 32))
 (segment (start 48.1237 43.5333) (end 47.207 44.45) (width 0.25) (layer B.Cu) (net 32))
 (segment (start 48.1237 35.88) (end 48.1237 43.2379) (width 0.25) (layer F.Cu) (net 32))
 (segment (start 48.979 35.88) (end 48.1237 35.88) (width 0.25) (layer F.Cu) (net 32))
 (via (at 48.1237 43.2379) (size 0.8) (layers F.Cu B.Cu) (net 32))
 (segment (start 45.832 52.07) (end 40.64 52.07) (width 0.25) (layer B.Cu) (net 20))
 (segment (start 45.757 49.53) (end 40.64 49.53) (width 0.25) (layer B.Cu) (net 21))
 (segment (start 45.757 46.99) (end 40.64 46.99) (width 0.25) (layer B.Cu) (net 22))
 (segment (start 45.757 44.45) (end 40.64 44.45) (width 0.25) (layer B.Cu) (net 23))
 (segment (start 52.23 46.736) (end 53.3053 46.736) (width 0.25) (layer F.Cu) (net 36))
 (segment (start 53.15 39.37) (end 53.3053 39.5253) (width 0.25) (layer F.Cu) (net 36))
 (segment (start 53.3053 39.5253) (end 53.3053 46.736) (width 0.25) (layer F.Cu) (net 36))
 (segment (start 54.8 36.322) (end 53.15 37.972) (width 0.25) (layer F.Cu) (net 36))
 (segment (start 53.15 37.972) (end 53.15 39.37) (width 0.25) (layer F.Cu) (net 36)))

